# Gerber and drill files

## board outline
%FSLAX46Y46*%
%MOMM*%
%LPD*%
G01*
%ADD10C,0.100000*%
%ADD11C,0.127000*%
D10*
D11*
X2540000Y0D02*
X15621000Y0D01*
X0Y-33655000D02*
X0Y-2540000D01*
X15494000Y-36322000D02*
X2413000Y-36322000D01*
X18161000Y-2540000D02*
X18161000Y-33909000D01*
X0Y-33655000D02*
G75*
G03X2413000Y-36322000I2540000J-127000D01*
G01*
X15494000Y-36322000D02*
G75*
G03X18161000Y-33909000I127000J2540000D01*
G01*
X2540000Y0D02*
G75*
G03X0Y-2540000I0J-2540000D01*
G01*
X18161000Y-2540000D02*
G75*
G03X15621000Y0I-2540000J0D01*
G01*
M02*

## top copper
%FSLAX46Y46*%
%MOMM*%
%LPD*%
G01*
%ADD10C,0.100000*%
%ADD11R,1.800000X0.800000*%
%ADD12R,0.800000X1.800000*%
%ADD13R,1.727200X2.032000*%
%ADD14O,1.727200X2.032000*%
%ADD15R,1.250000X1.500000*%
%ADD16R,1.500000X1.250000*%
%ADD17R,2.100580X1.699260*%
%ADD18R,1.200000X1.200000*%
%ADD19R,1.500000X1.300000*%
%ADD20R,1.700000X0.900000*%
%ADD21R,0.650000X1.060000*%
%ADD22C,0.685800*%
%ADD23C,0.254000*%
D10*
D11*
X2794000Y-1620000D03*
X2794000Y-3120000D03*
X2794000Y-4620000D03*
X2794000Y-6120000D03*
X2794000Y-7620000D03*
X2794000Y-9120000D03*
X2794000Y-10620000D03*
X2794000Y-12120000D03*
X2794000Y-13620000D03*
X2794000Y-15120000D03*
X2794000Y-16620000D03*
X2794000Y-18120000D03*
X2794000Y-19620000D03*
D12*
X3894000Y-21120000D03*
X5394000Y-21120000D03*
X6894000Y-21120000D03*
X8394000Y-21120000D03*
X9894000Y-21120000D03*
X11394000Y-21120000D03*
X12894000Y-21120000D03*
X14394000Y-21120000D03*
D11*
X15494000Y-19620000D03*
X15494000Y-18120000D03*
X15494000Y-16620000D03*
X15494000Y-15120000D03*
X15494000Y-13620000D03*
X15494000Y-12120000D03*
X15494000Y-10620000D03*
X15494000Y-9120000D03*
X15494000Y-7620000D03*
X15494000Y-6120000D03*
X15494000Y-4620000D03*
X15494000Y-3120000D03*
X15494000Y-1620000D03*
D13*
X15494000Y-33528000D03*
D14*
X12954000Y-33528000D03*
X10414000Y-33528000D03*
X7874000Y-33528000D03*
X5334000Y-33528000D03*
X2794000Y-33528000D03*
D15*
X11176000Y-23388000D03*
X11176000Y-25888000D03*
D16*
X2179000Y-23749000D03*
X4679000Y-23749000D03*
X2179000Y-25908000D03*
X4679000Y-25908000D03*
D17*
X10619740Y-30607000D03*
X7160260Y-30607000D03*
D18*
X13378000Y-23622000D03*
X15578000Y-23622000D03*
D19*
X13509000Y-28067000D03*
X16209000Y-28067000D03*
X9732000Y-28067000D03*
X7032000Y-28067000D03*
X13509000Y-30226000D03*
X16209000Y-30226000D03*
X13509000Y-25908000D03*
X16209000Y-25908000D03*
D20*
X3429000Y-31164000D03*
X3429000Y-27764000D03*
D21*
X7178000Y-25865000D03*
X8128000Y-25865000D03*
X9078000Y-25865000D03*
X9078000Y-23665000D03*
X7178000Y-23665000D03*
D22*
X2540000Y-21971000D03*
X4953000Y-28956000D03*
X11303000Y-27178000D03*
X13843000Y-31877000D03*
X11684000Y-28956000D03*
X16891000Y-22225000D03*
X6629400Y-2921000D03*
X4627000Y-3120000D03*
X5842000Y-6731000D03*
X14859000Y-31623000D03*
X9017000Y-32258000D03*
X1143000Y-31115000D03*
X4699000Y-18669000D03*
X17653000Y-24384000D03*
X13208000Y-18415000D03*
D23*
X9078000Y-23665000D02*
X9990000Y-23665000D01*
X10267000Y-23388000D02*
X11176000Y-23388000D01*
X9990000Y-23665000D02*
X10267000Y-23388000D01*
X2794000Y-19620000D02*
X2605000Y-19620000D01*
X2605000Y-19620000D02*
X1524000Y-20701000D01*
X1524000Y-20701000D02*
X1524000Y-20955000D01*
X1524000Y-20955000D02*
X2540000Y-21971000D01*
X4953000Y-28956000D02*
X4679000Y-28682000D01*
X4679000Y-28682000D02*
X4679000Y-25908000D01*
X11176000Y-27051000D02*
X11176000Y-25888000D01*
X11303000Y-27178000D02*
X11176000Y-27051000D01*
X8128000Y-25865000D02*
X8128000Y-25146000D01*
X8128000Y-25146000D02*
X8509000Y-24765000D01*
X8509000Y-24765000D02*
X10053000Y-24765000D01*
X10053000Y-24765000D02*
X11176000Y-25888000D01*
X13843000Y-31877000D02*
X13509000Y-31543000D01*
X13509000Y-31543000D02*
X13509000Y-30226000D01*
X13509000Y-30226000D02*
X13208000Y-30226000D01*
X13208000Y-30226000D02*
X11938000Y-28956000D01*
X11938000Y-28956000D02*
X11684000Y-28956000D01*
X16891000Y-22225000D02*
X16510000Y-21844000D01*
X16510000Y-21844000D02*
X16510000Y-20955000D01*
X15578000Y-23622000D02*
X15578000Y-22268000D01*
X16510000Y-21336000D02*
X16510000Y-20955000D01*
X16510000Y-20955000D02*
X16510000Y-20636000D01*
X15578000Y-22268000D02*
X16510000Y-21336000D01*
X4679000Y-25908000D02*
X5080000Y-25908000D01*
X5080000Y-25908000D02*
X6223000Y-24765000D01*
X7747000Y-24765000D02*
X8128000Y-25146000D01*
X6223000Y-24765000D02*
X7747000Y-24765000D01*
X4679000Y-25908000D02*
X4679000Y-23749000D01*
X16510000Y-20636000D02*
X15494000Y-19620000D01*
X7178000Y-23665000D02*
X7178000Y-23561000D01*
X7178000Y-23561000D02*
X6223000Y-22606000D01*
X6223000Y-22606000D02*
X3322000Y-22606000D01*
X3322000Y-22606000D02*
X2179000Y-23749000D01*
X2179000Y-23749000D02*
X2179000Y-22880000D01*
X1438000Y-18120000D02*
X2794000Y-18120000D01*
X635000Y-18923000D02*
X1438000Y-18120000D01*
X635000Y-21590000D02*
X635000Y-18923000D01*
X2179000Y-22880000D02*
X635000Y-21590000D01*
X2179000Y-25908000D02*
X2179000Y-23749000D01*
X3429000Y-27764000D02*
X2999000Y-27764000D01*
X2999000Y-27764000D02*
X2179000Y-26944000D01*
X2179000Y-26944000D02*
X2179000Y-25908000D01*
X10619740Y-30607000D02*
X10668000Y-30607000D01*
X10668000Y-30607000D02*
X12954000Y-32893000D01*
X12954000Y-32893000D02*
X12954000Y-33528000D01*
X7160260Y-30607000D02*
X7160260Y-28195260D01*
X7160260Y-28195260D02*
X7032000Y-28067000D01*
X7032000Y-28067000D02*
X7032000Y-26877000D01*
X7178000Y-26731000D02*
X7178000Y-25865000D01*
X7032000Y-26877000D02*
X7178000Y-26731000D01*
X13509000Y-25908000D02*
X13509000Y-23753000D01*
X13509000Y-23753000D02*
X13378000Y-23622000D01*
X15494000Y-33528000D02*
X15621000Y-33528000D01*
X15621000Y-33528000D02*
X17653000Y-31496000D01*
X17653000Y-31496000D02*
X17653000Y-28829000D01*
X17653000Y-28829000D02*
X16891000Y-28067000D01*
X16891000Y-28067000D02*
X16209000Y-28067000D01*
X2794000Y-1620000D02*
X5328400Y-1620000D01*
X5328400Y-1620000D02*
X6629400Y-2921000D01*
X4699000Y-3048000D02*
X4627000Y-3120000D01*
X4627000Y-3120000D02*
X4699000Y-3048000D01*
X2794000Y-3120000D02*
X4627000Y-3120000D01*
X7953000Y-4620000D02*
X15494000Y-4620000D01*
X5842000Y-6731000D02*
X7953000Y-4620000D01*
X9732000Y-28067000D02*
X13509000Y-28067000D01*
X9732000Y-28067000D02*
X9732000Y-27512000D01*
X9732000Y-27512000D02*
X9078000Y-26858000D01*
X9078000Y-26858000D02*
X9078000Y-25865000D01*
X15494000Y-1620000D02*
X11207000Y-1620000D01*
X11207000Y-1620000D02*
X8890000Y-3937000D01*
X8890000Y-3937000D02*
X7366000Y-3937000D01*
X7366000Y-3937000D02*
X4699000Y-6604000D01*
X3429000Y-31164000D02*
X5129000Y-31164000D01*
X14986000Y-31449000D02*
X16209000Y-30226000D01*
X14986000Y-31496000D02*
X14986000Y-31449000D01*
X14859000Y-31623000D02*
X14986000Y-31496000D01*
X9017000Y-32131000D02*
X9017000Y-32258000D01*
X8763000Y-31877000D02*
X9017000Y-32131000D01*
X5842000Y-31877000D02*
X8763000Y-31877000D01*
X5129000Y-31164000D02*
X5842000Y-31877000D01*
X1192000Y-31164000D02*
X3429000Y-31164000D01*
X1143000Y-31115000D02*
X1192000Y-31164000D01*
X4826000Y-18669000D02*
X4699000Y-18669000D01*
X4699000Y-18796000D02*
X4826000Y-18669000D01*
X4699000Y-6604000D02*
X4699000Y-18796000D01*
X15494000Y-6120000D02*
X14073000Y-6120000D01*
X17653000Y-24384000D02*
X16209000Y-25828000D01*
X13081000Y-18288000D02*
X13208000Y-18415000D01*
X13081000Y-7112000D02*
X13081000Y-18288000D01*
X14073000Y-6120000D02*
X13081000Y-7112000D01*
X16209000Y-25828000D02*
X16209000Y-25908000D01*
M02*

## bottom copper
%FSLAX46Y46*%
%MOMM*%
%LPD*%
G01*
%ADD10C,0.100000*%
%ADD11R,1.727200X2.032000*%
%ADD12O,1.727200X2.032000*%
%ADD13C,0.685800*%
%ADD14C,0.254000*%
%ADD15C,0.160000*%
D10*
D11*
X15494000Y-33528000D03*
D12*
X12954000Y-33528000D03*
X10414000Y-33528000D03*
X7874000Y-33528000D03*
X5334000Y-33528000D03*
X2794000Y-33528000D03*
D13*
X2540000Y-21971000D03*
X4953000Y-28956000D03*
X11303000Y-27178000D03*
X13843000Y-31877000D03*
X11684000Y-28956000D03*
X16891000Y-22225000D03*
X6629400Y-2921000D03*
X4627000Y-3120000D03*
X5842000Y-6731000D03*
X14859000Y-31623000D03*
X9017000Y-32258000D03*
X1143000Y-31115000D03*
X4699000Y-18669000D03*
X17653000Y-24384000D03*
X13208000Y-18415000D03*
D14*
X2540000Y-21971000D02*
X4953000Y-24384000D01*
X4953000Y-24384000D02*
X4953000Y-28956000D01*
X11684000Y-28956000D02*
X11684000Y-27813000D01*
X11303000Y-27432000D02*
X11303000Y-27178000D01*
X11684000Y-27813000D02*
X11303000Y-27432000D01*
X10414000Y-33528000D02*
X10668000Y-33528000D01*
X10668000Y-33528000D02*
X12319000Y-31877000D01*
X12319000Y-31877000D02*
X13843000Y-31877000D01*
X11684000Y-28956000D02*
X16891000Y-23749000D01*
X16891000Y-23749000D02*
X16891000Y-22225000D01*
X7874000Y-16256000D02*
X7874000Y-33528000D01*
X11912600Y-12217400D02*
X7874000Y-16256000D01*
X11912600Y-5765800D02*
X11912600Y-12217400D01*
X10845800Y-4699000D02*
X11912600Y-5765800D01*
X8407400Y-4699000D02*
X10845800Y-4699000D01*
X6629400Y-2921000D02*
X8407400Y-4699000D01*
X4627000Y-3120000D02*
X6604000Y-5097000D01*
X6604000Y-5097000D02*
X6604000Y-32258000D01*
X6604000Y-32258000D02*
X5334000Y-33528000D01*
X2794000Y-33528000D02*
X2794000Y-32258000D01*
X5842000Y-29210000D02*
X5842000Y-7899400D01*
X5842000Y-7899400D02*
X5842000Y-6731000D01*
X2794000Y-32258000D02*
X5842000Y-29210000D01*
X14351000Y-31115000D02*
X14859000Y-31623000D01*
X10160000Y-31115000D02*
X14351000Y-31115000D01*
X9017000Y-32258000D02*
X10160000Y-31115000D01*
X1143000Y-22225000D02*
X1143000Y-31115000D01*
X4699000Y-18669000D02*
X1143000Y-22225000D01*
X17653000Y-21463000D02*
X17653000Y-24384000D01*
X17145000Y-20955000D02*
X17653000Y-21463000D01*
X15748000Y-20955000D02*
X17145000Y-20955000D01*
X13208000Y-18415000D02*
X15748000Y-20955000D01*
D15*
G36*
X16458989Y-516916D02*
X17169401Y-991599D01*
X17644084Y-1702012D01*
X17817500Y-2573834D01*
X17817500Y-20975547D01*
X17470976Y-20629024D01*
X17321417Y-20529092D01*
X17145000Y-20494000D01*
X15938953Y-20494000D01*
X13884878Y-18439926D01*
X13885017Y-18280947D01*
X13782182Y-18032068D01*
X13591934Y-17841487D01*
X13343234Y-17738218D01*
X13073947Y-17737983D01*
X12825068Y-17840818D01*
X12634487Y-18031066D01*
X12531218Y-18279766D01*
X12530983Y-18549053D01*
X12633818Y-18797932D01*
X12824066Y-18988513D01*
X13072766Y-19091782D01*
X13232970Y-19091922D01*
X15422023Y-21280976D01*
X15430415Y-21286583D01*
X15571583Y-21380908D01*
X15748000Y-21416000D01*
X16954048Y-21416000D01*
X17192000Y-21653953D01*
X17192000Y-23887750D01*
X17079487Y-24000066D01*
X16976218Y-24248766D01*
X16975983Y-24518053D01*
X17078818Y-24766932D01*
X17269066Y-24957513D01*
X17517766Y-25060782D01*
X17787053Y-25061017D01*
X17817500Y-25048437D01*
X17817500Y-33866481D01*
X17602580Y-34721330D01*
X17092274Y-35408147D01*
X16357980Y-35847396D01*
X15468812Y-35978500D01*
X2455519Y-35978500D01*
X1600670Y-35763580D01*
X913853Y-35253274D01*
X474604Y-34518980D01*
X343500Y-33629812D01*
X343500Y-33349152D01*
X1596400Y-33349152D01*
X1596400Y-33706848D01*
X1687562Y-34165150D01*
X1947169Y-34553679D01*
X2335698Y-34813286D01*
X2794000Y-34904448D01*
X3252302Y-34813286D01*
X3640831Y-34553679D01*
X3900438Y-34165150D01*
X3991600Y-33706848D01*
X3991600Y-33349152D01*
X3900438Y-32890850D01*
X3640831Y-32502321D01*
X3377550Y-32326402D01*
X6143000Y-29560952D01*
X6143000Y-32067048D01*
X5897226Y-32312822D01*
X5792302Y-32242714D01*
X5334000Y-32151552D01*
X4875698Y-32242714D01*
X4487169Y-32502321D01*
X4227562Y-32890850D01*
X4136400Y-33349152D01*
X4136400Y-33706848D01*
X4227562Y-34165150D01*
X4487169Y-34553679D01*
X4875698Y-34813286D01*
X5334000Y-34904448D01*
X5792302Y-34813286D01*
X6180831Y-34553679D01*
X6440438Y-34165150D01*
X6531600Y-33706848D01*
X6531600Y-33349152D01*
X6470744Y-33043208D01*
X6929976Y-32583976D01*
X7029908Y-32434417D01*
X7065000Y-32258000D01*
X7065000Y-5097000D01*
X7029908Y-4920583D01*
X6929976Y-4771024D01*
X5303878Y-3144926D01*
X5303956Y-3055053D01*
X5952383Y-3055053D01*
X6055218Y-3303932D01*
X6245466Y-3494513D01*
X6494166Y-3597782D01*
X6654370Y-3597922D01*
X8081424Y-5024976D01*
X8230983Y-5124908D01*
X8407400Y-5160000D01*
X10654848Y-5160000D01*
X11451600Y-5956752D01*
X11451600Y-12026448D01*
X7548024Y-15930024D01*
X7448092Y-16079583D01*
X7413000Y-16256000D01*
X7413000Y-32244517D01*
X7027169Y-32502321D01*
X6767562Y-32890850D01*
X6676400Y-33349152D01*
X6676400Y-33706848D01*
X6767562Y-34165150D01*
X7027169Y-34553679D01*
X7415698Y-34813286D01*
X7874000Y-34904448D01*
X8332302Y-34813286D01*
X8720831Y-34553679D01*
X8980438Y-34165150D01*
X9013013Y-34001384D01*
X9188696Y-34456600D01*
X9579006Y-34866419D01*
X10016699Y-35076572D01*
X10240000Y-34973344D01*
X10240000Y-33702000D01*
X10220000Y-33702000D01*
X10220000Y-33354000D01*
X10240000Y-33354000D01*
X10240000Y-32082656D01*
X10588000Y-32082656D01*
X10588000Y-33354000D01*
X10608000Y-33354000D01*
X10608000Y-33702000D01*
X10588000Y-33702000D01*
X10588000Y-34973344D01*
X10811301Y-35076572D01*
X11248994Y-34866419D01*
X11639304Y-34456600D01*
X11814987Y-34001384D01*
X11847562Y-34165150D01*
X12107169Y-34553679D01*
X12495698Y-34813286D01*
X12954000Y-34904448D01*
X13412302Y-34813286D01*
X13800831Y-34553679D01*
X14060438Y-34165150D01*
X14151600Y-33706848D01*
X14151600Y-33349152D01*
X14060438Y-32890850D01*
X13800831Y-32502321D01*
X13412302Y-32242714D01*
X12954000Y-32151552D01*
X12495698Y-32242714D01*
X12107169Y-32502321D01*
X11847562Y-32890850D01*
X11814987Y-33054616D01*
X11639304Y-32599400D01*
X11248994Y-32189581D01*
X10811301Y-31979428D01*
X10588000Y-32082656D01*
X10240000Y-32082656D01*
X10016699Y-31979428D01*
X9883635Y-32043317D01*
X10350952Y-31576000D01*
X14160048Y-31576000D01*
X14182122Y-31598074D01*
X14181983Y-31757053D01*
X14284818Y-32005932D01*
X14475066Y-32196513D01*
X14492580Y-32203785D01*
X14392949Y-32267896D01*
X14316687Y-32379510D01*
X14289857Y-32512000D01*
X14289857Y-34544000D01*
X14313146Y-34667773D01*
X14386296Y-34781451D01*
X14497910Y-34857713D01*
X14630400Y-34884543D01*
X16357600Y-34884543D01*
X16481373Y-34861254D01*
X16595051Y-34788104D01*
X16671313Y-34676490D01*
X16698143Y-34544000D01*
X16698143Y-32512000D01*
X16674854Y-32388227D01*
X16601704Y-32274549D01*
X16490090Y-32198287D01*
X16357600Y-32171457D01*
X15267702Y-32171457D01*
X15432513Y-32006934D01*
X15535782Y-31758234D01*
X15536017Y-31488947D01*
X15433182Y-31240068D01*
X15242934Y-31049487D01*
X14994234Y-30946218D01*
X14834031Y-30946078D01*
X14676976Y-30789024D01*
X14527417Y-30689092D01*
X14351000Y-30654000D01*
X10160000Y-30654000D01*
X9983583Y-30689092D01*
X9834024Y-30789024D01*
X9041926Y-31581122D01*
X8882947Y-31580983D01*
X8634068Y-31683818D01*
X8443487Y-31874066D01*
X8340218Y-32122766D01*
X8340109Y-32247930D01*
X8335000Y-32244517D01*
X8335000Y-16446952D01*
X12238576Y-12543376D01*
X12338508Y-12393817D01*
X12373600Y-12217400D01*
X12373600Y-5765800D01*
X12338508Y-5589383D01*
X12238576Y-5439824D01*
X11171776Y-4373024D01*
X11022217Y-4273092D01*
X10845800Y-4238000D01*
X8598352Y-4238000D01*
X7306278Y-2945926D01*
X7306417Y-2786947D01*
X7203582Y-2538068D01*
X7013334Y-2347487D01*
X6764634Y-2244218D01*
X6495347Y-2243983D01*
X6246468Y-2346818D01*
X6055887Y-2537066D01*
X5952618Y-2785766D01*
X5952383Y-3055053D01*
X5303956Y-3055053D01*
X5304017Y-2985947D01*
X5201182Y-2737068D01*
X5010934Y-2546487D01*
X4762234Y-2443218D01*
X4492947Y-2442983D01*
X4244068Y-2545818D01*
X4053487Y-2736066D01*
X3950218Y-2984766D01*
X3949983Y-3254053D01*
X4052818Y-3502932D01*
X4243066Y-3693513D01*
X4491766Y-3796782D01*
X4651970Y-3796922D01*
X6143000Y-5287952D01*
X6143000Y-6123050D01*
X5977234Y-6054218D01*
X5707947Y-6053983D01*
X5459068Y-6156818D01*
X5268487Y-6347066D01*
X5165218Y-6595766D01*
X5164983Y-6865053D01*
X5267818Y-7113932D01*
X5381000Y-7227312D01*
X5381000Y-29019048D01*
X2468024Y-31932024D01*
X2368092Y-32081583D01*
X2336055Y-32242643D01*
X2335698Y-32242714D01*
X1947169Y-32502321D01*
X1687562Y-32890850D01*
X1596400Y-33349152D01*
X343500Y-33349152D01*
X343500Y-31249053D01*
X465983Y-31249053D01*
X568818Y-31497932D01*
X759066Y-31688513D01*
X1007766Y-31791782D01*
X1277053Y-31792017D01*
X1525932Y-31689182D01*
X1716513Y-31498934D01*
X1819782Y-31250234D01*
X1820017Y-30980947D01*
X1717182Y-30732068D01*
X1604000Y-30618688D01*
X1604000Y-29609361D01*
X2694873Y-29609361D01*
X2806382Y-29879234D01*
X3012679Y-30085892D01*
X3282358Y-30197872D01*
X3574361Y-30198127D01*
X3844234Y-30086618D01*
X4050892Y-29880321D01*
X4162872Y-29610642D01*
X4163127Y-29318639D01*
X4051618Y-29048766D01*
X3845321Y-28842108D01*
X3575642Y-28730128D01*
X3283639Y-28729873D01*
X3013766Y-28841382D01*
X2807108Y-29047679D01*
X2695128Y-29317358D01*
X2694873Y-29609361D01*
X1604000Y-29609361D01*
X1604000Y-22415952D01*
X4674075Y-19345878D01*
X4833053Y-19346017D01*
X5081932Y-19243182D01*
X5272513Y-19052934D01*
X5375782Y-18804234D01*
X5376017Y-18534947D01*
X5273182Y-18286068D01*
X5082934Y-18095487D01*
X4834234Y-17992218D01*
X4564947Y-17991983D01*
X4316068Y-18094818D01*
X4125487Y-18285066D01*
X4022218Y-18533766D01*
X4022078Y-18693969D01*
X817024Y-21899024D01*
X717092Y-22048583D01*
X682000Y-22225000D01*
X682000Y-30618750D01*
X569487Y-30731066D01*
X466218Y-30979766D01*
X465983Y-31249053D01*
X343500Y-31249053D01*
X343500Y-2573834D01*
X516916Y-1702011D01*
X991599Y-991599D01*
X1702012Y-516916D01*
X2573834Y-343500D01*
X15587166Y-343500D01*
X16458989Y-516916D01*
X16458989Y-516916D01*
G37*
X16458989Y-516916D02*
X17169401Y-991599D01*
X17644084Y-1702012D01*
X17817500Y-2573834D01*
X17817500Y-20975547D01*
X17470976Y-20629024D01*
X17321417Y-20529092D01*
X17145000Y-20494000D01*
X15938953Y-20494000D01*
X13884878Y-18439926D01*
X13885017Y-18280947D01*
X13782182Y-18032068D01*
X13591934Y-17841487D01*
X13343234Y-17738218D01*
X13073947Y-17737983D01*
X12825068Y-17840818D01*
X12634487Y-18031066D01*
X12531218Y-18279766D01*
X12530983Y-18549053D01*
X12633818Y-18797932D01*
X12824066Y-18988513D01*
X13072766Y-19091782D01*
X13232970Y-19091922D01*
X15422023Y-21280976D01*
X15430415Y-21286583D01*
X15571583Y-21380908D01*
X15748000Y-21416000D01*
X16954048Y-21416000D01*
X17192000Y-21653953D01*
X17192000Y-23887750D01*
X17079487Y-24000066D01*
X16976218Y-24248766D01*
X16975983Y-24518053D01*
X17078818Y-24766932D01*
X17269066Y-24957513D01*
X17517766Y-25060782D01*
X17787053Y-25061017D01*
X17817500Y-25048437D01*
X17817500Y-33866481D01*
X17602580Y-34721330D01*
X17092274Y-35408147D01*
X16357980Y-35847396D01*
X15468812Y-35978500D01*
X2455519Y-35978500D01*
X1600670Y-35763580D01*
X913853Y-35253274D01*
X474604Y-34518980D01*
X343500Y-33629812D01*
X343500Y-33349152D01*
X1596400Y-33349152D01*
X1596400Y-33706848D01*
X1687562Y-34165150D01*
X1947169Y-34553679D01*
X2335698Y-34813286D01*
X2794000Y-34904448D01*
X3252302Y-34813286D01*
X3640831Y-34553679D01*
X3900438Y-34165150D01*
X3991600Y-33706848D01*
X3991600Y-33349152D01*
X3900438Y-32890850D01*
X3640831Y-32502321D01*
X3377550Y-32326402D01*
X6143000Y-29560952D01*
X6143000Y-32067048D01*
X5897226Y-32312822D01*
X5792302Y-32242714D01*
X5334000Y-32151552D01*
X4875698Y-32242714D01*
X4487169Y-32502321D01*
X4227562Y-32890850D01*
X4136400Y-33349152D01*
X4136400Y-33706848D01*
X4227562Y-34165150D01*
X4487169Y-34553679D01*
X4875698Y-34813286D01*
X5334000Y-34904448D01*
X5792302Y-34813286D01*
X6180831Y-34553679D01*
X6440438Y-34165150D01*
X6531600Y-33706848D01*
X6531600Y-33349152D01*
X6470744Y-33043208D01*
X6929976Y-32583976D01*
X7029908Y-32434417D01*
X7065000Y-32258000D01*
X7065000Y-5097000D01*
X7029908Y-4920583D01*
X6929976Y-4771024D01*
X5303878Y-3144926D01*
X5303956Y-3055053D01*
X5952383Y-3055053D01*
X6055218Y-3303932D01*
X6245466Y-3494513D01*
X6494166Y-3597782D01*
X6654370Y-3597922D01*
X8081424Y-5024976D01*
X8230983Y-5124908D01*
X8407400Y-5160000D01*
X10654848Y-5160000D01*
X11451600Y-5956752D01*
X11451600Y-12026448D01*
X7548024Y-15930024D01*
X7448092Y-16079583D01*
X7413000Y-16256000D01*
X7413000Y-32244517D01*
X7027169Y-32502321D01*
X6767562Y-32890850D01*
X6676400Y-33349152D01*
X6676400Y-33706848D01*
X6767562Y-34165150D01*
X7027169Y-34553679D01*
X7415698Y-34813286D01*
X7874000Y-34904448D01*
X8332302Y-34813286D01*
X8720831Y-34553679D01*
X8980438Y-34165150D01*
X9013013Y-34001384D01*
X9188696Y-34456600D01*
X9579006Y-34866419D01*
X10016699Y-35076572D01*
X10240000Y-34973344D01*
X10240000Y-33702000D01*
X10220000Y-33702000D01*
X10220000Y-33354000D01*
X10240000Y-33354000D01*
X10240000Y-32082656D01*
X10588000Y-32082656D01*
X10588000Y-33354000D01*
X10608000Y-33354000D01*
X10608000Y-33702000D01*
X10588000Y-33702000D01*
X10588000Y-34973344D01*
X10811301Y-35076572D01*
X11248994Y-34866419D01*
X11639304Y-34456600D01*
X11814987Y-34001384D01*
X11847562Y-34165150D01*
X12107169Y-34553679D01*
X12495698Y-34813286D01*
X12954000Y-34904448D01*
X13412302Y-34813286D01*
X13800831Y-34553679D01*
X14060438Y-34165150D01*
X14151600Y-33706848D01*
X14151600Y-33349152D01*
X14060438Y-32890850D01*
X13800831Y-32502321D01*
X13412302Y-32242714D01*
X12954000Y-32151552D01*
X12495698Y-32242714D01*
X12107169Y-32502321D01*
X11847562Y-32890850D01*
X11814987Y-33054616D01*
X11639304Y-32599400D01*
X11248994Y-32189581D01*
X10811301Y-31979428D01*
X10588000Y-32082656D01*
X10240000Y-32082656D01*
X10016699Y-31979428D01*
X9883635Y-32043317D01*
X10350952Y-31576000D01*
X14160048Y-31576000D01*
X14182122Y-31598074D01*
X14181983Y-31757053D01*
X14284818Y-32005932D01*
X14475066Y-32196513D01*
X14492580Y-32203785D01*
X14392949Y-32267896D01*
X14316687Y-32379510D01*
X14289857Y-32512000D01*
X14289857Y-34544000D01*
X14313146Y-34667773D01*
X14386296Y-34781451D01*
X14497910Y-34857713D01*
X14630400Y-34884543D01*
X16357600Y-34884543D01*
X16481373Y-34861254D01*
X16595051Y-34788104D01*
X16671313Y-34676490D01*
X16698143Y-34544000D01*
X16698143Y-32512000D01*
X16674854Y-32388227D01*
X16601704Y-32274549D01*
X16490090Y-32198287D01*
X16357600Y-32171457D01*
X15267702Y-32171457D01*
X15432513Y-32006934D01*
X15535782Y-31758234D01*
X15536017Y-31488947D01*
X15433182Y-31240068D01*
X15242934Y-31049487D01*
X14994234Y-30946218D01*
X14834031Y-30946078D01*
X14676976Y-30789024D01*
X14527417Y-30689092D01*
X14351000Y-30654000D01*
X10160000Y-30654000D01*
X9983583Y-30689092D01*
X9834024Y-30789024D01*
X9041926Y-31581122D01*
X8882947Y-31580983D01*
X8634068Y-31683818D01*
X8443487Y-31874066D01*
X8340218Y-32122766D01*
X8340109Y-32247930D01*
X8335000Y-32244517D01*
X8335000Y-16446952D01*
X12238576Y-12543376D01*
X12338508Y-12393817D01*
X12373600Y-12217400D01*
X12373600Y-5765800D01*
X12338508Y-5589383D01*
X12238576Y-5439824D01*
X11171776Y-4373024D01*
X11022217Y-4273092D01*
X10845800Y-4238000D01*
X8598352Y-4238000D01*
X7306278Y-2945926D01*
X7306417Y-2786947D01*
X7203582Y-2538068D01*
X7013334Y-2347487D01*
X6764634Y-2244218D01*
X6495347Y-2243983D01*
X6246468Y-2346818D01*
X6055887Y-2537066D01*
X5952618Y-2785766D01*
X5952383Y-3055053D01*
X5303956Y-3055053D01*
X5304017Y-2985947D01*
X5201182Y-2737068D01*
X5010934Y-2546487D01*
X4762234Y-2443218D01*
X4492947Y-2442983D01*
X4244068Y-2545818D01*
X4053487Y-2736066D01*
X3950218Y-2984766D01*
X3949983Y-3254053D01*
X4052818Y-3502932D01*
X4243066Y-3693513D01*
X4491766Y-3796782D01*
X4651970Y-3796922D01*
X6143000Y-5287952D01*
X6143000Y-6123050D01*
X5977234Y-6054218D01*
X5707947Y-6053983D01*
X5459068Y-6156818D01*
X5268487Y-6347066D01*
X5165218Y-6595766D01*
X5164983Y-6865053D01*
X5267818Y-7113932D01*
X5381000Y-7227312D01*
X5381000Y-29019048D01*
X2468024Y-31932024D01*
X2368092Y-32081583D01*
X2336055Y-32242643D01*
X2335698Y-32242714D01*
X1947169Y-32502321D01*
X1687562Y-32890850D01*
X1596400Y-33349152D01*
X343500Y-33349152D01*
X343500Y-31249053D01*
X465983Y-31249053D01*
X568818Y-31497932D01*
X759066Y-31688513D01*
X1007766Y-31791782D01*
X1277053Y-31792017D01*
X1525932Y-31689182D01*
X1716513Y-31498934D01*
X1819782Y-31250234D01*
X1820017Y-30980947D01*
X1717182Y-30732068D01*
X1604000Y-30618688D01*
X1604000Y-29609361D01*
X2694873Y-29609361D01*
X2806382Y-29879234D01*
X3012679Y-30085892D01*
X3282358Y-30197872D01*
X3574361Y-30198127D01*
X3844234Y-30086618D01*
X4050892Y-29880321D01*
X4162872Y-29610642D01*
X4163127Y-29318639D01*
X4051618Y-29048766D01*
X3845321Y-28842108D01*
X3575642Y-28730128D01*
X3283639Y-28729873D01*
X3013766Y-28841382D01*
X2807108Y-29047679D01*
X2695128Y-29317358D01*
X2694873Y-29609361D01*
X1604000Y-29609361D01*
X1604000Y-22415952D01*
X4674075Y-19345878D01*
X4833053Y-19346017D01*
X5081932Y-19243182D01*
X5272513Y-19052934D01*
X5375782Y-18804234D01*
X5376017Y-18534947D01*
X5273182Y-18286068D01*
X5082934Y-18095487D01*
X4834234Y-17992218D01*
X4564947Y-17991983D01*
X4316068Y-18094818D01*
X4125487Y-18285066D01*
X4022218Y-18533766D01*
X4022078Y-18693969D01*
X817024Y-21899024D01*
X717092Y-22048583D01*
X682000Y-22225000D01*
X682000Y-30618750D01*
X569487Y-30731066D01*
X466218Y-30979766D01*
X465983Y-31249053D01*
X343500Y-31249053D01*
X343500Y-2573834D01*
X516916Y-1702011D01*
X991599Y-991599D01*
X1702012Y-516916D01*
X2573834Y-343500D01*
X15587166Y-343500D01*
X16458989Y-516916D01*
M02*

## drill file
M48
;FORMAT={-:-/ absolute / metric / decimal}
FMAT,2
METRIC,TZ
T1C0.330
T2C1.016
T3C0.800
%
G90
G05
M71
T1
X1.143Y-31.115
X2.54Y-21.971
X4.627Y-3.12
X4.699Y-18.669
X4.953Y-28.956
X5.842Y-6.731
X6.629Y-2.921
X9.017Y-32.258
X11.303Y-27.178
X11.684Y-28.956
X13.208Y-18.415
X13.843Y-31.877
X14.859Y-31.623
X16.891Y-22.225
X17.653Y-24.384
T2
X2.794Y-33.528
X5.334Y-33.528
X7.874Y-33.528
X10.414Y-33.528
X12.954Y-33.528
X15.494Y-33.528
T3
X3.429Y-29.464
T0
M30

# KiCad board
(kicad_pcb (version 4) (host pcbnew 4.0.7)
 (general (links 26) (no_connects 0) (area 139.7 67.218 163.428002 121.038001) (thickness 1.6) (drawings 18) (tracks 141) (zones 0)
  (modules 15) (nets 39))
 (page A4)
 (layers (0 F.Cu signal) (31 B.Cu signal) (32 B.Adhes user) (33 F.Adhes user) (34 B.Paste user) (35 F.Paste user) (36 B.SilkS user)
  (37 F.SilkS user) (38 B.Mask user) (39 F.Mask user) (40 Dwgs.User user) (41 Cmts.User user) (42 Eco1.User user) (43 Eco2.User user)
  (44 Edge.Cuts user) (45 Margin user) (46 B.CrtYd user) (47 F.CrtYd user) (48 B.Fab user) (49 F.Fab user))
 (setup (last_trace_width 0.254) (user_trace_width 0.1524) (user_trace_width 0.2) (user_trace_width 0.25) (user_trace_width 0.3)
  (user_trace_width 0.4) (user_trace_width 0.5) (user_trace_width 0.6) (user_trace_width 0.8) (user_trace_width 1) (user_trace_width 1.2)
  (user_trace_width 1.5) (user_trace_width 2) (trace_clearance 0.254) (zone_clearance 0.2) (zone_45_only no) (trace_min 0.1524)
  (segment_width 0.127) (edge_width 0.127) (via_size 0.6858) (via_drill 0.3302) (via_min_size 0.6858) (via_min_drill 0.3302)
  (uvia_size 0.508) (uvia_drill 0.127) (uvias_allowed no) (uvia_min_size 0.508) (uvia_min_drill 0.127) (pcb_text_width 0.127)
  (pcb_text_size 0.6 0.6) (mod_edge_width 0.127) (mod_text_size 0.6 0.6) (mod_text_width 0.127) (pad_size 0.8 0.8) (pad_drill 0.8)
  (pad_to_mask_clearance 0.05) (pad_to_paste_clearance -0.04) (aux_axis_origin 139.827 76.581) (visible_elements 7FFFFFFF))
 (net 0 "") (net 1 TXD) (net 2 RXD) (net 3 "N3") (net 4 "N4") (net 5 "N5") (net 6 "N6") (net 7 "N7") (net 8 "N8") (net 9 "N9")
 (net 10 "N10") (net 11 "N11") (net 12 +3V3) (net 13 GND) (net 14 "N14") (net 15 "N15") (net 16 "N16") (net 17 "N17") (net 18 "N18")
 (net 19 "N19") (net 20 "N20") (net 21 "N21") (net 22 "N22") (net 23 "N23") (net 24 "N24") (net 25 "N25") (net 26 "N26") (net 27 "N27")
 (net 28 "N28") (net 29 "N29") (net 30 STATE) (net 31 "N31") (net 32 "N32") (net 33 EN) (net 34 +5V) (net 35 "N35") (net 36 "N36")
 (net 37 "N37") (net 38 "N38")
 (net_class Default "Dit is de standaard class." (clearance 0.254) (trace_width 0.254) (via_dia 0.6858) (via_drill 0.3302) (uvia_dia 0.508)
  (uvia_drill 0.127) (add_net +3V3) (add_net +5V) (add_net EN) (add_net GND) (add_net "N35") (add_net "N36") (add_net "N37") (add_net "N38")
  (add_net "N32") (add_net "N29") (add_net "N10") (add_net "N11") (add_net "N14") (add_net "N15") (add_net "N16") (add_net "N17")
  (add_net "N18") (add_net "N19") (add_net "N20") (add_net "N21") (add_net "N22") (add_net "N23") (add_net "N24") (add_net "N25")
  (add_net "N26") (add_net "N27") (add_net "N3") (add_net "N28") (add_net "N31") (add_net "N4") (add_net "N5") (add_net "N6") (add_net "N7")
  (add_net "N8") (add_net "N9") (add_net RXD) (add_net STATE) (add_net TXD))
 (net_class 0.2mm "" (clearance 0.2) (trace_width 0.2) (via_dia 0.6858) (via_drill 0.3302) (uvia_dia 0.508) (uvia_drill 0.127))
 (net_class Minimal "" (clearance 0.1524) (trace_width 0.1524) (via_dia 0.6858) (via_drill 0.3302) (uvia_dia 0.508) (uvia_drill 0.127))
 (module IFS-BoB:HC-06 (layer F.Cu) (at 148.971 84.201)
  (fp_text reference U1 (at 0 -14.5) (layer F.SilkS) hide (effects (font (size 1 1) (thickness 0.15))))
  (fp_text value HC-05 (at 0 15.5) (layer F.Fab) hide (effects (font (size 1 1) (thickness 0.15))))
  (pad 1 smd rect (at -6.35 -6) (size 1.8 0.8) (layers F.Cu F.Paste F.Mask) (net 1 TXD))
  (pad 2 smd rect (at -6.35 -4.5) (size 1.8 0.8) (layers F.Cu F.Paste F.Mask) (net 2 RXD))
  (pad 3 smd rect (at -6.35 -3) (size 1.8 0.8) (layers F.Cu F.Paste F.Mask) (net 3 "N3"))
  (pad 4 smd rect (at -6.35 -1.5) (size 1.8 0.8) (layers F.Cu F.Paste F.Mask) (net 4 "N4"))
  (pad 5 smd rect (at -6.35 0) (size 1.8 0.8) (layers F.Cu F.Paste F.Mask) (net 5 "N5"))
  (pad 6 smd rect (at -6.35 1.5) (size 1.8 0.8) (layers F.Cu F.Paste F.Mask) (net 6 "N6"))
  (pad 7 smd rect (at -6.35 3) (size 1.8 0.8) (layers F.Cu F.Paste F.Mask) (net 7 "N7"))
  (pad 8 smd rect (at -6.35 4.5) (size 1.8 0.8) (layers F.Cu F.Paste F.Mask) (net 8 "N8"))
  (pad 9 smd rect (at -6.35 6) (size 1.8 0.8) (layers F.Cu F.Paste F.Mask) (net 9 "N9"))
  (pad 10 smd rect (at -6.35 7.5) (size 1.8 0.8) (layers F.Cu F.Paste F.Mask) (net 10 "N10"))
  (pad 11 smd rect (at -6.35 9) (size 1.8 0.8) (layers F.Cu F.Paste F.Mask) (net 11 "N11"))
  (pad 12 smd rect (at -6.35 10.5) (size 1.8 0.8) (layers F.Cu F.Paste F.Mask) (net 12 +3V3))
  (pad 13 smd rect (at -6.35 12) (size 1.8 0.8) (layers F.Cu F.Paste F.Mask) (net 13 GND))
  (pad 14 smd rect (at -5.25 13.5) (size 0.8 1.8) (layers F.Cu F.Paste F.Mask) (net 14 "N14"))
  (pad 15 smd rect (at -3.75 13.5) (size 0.8 1.8) (layers F.Cu F.Paste F.Mask) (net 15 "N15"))
  (pad 16 smd rect (at -2.25 13.5) (size 0.8 1.8) (layers F.Cu F.Paste F.Mask) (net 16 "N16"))
  (pad 17 smd rect (at -0.75 13.5) (size 0.8 1.8) (layers F.Cu F.Paste F.Mask) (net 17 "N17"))
  (pad 18 smd rect (at 0.75 13.5) (size 0.8 1.8) (layers F.Cu F.Paste F.Mask))
  (pad 19 smd rect (at 2.25 13.5) (size 0.8 1.8) (layers F.Cu F.Paste F.Mask) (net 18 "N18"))
  (pad 20 smd rect (at 3.75 13.5) (size 0.8 1.8) (layers F.Cu F.Paste F.Mask) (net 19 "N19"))
  (pad 21 smd rect (at 5.25 13.5) (size 0.8 1.8) (layers F.Cu F.Paste F.Mask) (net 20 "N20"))
  (pad 22 smd rect (at 6.35 12) (size 1.8 0.8) (layers F.Cu F.Paste F.Mask) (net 13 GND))
  (pad 23 smd rect (at 6.35 10.5) (size 1.8 0.8) (layers F.Cu F.Paste F.Mask) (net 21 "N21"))
  (pad 24 smd rect (at 6.35 9) (size 1.8 0.8) (layers F.Cu F.Paste F.Mask) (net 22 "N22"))
  (pad 25 smd rect (at 6.35 7.5) (size 1.8 0.8) (layers F.Cu F.Paste F.Mask) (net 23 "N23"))
  (pad 26 smd rect (at 6.35 6) (size 1.8 0.8) (layers F.Cu F.Paste F.Mask) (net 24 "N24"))
  (pad 27 smd rect (at 6.35 4.5) (size 1.8 0.8) (layers F.Cu F.Paste F.Mask) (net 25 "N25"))
  (pad 28 smd rect (at 6.35 3) (size 1.8 0.8) (layers F.Cu F.Paste F.Mask) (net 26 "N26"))
  (pad 29 smd rect (at 6.35 1.5) (size 1.8 0.8) (layers F.Cu F.Paste F.Mask) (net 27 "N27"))
  (pad 30 smd rect (at 6.35 0) (size 1.8 0.8) (layers F.Cu F.Paste F.Mask) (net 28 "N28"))
  (pad 31 smd rect (at 6.35 -1.5) (size 1.8 0.8) (layers F.Cu F.Paste F.Mask) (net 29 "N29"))
  (pad 32 smd rect (at 6.35 -3) (size 1.8 0.8) (layers F.Cu F.Paste F.Mask) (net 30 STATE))
  (pad 33 smd rect (at 6.35 -4.5) (size 1.8 0.8) (layers F.Cu F.Paste F.Mask) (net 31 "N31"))
  (pad 34 smd rect (at 6.35 -6) (size 1.8 0.8) (layers F.Cu F.Paste F.Mask) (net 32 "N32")))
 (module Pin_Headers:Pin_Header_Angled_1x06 (layer F.Cu) (at 155.321 110.109 270)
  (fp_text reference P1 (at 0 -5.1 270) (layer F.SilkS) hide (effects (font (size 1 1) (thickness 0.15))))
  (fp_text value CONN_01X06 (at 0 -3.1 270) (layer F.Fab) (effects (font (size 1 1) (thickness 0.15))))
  (pad 1 thru_hole rect (at 0 0 270) (size 2.032 1.7272) (drill 1.016) (layers *.Cu *.Mask) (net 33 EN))
  (pad 2 thru_hole oval (at 0 2.54 270) (size 2.032 1.7272) (drill 1.016) (layers *.Cu *.Mask) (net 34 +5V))
  (pad 3 thru_hole oval (at 0 5.08 270) (size 2.032 1.7272) (drill 1.016) (layers *.Cu *.Mask) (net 13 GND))
  (pad 4 thru_hole oval (at 0 7.62 270) (size 2.032 1.7272) (drill 1.016) (layers *.Cu *.Mask) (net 1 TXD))
  (pad 5 thru_hole oval (at 0 10.16 270) (size 2.032 1.7272) (drill 1.016) (layers *.Cu *.Mask) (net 2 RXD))
  (pad 6 thru_hole oval (at 0 12.7 270) (size 2.032 1.7272) (drill 1.016) (layers *.Cu *.Mask) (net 30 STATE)))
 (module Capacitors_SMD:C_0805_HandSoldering (layer F.Cu) (at 151.003 101.219 270)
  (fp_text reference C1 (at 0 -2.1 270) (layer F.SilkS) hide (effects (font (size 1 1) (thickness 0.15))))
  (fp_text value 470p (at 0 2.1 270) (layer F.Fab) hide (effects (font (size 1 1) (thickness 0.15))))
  (pad 1 smd rect (at -1.25 0 270) (size 1.5 1.25) (layers F.Cu F.Paste F.Mask) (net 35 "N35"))
  (pad 2 smd rect (at 1.25 0 270) (size 1.5 1.25) (layers F.Cu F.Paste F.Mask) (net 13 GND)))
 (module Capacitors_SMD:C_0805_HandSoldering (layer F.Cu) (at 143.256 100.33)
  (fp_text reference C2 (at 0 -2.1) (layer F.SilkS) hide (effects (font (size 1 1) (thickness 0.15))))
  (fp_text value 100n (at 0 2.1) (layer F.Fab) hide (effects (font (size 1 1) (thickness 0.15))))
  (pad 1 smd rect (at -1.25 0) (size 1.5 1.25) (layers F.Cu F.Paste F.Mask) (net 12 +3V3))
  (pad 2 smd rect (at 1.25 0) (size 1.5 1.25) (layers F.Cu F.Paste F.Mask) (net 13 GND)))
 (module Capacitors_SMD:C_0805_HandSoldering (layer F.Cu) (at 143.256 102.489)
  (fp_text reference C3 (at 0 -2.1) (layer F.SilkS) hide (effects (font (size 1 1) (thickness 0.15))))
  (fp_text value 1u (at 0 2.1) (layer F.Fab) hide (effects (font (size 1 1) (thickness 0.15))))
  (pad 1 smd rect (at -1.25 0) (size 1.5 1.25) (layers F.Cu F.Paste F.Mask) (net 12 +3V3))
  (pad 2 smd rect (at 1.25 0) (size 1.5 1.25) (layers F.Cu F.Paste F.Mask) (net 13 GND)))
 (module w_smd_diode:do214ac (layer F.Cu) (at 148.717 107.188)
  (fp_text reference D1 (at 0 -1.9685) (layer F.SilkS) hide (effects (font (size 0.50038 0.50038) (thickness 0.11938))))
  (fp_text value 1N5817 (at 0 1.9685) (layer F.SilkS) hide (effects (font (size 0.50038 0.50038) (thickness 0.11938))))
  (pad 2 smd rect (at 1.72974 0) (size 2.10058 1.69926) (layers F.Cu F.Paste F.Mask) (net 34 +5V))
  (pad 1 smd rect (at -1.72974 0) (size 2.10058 1.69926) (layers F.Cu F.Paste F.Mask) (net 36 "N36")))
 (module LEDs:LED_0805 (layer F.Cu) (at 154.305 100.203 180)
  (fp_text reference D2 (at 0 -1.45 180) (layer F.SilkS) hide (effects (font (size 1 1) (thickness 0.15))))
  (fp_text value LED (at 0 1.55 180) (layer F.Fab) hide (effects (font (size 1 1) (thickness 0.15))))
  (pad 2 smd rect (at 1.1 0) (size 1.2 1.2) (layers F.Cu F.Paste F.Mask) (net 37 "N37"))
  (pad 1 smd rect (at -1.1 0) (size 1.2 1.2) (layers F.Cu F.Paste F.Mask) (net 13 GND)))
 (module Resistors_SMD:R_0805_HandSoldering (layer F.Cu) (at 154.686 104.648)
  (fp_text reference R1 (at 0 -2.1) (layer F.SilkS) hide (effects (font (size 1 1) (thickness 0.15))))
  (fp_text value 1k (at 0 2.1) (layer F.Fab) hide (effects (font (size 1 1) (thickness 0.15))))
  (pad 1 smd rect (at -1.35 0) (size 1.5 1.3) (layers F.Cu F.Paste F.Mask) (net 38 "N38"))
  (pad 2 smd rect (at 1.35 0) (size 1.5 1.3) (layers F.Cu F.Paste F.Mask) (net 33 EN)))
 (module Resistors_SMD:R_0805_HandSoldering (layer F.Cu) (at 148.209 104.648 180)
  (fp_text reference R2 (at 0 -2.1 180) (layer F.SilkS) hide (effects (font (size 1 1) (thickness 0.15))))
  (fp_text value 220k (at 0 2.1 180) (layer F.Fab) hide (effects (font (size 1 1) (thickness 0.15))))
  (pad 1 smd rect (at -1.35 0 180) (size 1.5 1.3) (layers F.Cu F.Paste F.Mask) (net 38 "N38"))
  (pad 2 smd rect (at 1.35 0 180) (size 1.5 1.3) (layers F.Cu F.Paste F.Mask) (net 36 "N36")))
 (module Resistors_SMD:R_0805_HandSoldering (layer F.Cu) (at 154.686 106.807)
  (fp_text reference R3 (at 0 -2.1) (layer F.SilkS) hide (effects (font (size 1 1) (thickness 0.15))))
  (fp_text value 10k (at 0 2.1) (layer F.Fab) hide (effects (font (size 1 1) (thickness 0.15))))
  (pad 1 smd rect (at -1.35 0) (size 1.5 1.3) (layers F.Cu F.Paste F.Mask) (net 13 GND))
  (pad 2 smd rect (at 1.35 0) (size 1.5 1.3) (layers F.Cu F.Paste F.Mask) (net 32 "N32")))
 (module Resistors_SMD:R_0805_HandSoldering (layer F.Cu) (at 154.686 102.489)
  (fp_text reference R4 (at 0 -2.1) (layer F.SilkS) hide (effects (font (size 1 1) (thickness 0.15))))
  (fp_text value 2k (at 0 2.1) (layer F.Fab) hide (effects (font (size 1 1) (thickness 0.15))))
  (pad 1 smd rect (at -1.35 0) (size 1.5 1.3) (layers F.Cu F.Paste F.Mask) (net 37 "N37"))
  (pad 2 smd rect (at 1.35 0) (size 1.5 1.3) (layers F.Cu F.Paste F.Mask) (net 29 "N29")))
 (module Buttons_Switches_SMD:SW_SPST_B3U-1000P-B (layer F.Cu) (at 143.256 106.045 90)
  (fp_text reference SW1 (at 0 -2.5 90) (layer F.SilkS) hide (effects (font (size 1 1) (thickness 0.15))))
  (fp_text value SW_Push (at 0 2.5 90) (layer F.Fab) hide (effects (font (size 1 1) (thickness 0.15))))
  (pad 1 smd rect (at -1.7 0 90) (size 0.9 1.7) (layers F.Cu F.Paste F.Mask) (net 32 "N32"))
  (pad 2 smd rect (at 1.7 0 90) (size 0.9 1.7) (layers F.Cu F.Paste F.Mask) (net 12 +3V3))
  (pad "" np_thru_hole circle (at 0 0 90) (size 0.8 0.8) (drill 0.8) (layers *.Cu *.Mask)))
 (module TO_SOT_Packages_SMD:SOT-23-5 (layer F.Cu) (at 147.955 101.346 90)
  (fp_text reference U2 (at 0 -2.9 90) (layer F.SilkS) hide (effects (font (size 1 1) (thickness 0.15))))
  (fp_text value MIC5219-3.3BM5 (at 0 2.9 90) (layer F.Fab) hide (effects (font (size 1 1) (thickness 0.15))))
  (pad 1 smd rect (at -1.1 -0.95 90) (size 1.06 0.65) (layers F.Cu F.Paste F.Mask) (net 36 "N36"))
  (pad 2 smd rect (at -1.1 0 90) (size 1.06 0.65) (layers F.Cu F.Paste F.Mask) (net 13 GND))
  (pad 3 smd rect (at -1.1 0.95 90) (size 1.06 0.65) (layers F.Cu F.Paste F.Mask) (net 38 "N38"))
  (pad 4 smd rect (at 1.1 0.95 90) (size 1.06 0.65) (layers F.Cu F.Paste F.Mask) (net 35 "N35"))
  (pad 5 smd rect (at 1.1 -0.95 90) (size 1.06 0.65) (layers F.Cu F.Paste F.Mask) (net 12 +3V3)))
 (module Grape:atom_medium (layer B.Cu) (at 148.9964 87.376 180)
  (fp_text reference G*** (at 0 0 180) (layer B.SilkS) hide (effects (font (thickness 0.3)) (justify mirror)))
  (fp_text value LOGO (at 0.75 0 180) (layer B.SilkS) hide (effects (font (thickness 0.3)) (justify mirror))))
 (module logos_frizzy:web (layer B.Cu) (at 148.9456 95.3897 180)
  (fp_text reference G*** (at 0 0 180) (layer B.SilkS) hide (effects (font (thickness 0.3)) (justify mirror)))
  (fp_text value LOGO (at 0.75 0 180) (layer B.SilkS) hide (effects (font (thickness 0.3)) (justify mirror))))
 (gr_line (start 142.367 76.581) (end 155.448 76.581) (angle 90) (layer Edge.Cuts) (width 0.127))
 (gr_line (start 139.827 110.236) (end 139.827 79.121) (angle 90) (layer Edge.Cuts) (width 0.127))
 (gr_line (start 155.321 112.903) (end 142.24 112.903) (angle 90) (layer Edge.Cuts) (width 0.127))
 (gr_line (start 157.988 79.121) (end 157.988 110.49) (angle 90) (layer Edge.Cuts) (width 0.127))
 (gr_arc (start 142.367 110.363) (end 142.24 112.903) (angle 90) (layer Edge.Cuts) (width 0.127))
 (gr_arc (start 155.448 110.363) (end 157.988 110.49) (angle 90) (layer Edge.Cuts) (width 0.127))
 (gr_arc (start 142.367 79.121) (end 139.827 79.121) (angle 90) (layer Edge.Cuts) (width 0.127))
 (gr_arc (start 155.448 79.121) (end 155.448 76.581) (angle 90) (layer Edge.Cuts) (width 0.127))
 (segment (start 148.905 100.246) (end 149.817 100.246) (width 0.254) (layer F.Cu) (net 35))
 (segment (start 150.094 99.969) (end 151.003 99.969) (width 0.254) (layer F.Cu) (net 35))
 (segment (start 149.817 100.246) (end 150.094 99.969) (width 0.254) (layer F.Cu) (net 35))
 (segment (start 142.621 96.201) (end 142.432 96.201) (width 0.254) (layer F.Cu) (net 13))
 (segment (start 142.432 96.201) (end 141.351 97.282) (width 0.254) (layer F.Cu) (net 13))
 (segment (start 141.351 97.282) (end 141.351 97.536) (width 0.254) (layer F.Cu) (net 13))
 (segment (start 141.351 97.536) (end 142.367 98.552) (width 0.254) (layer F.Cu) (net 13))
 (via (at 142.367 98.552) (size 0.6858) (drill 0.3302) (layers F.Cu B.Cu) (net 13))
 (segment (start 142.367 98.552) (end 144.78 100.965) (width 0.254) (layer B.Cu) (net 13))
 (segment (start 144.78 100.965) (end 144.78 105.537) (width 0.254) (layer B.Cu) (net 13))
 (via (at 144.78 105.537) (size 0.6858) (drill 0.3302) (layers F.Cu B.Cu) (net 13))
 (segment (start 144.78 105.537) (end 144.506 105.263) (width 0.254) (layer F.Cu) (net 13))
 (segment (start 144.506 105.263) (end 144.506 102.489) (width 0.254) (layer F.Cu) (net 13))
 (segment (start 151.511 105.537) (end 151.511 104.394) (width 0.254) (layer B.Cu) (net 13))
 (segment (start 151.003 103.632) (end 151.003 102.469) (width 0.254) (layer F.Cu) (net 13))
 (segment (start 151.13 103.759) (end 151.003 103.632) (width 0.254) (layer F.Cu) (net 13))
 (via (at 151.13 103.759) (size 0.6858) (drill 0.3302) (layers F.Cu B.Cu) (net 13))
 (segment (start 151.13 104.013) (end 151.13 103.759) (width 0.254) (layer B.Cu) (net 13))
 (segment (start 151.511 104.394) (end 151.13 104.013) (width 0.254) (layer B.Cu) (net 13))
 (segment (start 147.955 102.446) (end 147.955 101.727) (width 0.254) (layer F.Cu) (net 13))
 (segment (start 147.955 101.727) (end 148.336 101.346) (width 0.254) (layer F.Cu) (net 13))
 (segment (start 148.336 101.346) (end 149.88 101.346) (width 0.254) (layer F.Cu) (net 13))
 (segment (start 149.88 101.346) (end 151.003 102.469) (width 0.254) (layer F.Cu) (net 13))
 (segment (start 150.241 110.109) (end 150.495 110.109) (width 0.254) (layer B.Cu) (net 13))
 (segment (start 150.495 110.109) (end 152.146 108.458) (width 0.254) (layer B.Cu) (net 13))
 (segment (start 152.146 108.458) (end 153.67 108.458) (width 0.254) (layer B.Cu) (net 13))
 (via (at 153.67 108.458) (size 0.6858) (drill 0.3302) (layers F.Cu B.Cu) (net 13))
 (segment (start 153.67 108.458) (end 153.336 108.124) (width 0.254) (layer F.Cu) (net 13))
 (segment (start 153.336 108.124) (end 153.336 106.807) (width 0.254) (layer F.Cu) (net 13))
 (segment (start 153.336 106.807) (end 153.035 106.807) (width 0.254) (layer F.Cu) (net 13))
 (segment (start 153.035 106.807) (end 151.765 105.537) (width 0.254) (layer F.Cu) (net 13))
 (segment (start 151.765 105.537) (end 151.511 105.537) (width 0.254) (layer F.Cu) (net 13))
 (via (at 151.511 105.537) (size 0.6858) (drill 0.3302) (layers F.Cu B.Cu) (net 13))
 (segment (start 151.511 105.537) (end 156.718 100.33) (width 0.254) (layer B.Cu) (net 13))
 (segment (start 156.718 100.33) (end 156.718 98.806) (width 0.254) (layer B.Cu) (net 13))
 (via (at 156.718 98.806) (size 0.6858) (drill 0.3302) (layers F.Cu B.Cu) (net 13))
 (segment (start 156.718 98.806) (end 156.337 98.425) (width 0.254) (layer F.Cu) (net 13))
 (segment (start 156.337 98.425) (end 156.337 97.536) (width 0.254) (layer F.Cu) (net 13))
 (segment (start 155.405 100.203) (end 155.405 98.849) (width 0.254) (layer F.Cu) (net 13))
 (segment (start 156.337 97.917) (end 156.337 97.536) (width 0.254) (layer F.Cu) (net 13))
 (segment (start 156.337 97.536) (end 156.337 97.217) (width 0.254) (layer F.Cu) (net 13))
 (segment (start 155.405 98.849) (end 156.337 97.917) (width 0.254) (layer F.Cu) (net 13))
 (segment (start 144.506 102.489) (end 144.907 102.489) (width 0.254) (layer F.Cu) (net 13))
 (segment (start 144.907 102.489) (end 146.05 101.346) (width 0.254) (layer F.Cu) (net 13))
 (segment (start 147.574 101.346) (end 147.955 101.727) (width 0.254) (layer F.Cu) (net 13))
 (segment (start 146.05 101.346) (end 147.574 101.346) (width 0.254) (layer F.Cu) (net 13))
 (segment (start 144.506 102.489) (end 144.506 100.33) (width 0.254) (layer F.Cu) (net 13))
 (segment (start 156.337 97.217) (end 155.321 96.201) (width 0.254) (layer F.Cu) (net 13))
 (segment (start 147.005 100.246) (end 147.005 100.142) (width 0.254) (layer F.Cu) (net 12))
 (segment (start 147.005 100.142) (end 146.05 99.187) (width 0.254) (layer F.Cu) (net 12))
 (segment (start 146.05 99.187) (end 143.149 99.187) (width 0.254) (layer F.Cu) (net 12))
 (segment (start 143.149 99.187) (end 142.006 100.33) (width 0.254) (layer F.Cu) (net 12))
 (segment (start 142.006 100.33) (end 142.006 99.461) (width 0.254) (layer F.Cu) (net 12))
 (segment (start 141.265 94.701) (end 142.621 94.701) (width 0.254) (layer F.Cu) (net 12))
 (segment (start 140.462 95.504) (end 141.265 94.701) (width 0.254) (layer F.Cu) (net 12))
 (segment (start 140.462 98.171) (end 140.462 95.504) (width 0.254) (layer F.Cu) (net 12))
 (segment (start 142.006 99.461) (end 140.462 98.171) (width 0.254) (layer F.Cu) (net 12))
 (segment (start 142.006 102.489) (end 142.006 100.33) (width 0.254) (layer F.Cu) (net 12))
 (segment (start 143.256 104.345) (end 142.826 104.345) (width 0.254) (layer F.Cu) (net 12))
 (segment (start 142.826 104.345) (end 142.006 103.525) (width 0.254) (layer F.Cu) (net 12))
 (segment (start 142.006 103.525) (end 142.006 102.489) (width 0.254) (layer F.Cu) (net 12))
 (segment (start 150.44674 107.188) (end 150.495 107.188) (width 0.254) (layer F.Cu) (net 34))
 (segment (start 150.495 107.188) (end 152.781 109.474) (width 0.254) (layer F.Cu) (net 34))
 (segment (start 152.781 109.474) (end 152.781 110.109) (width 0.254) (layer F.Cu) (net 34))
 (segment (start 146.98726 107.188) (end 146.98726 104.77626) (width 0.254) (layer F.Cu) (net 36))
 (segment (start 146.98726 104.77626) (end 146.859 104.648) (width 0.254) (layer F.Cu) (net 36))
 (segment (start 146.859 104.648) (end 146.859 103.458) (width 0.254) (layer F.Cu) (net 36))
 (segment (start 147.005 103.312) (end 147.005 102.446) (width 0.254) (layer F.Cu) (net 36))
 (segment (start 146.859 103.458) (end 147.005 103.312) (width 0.254) (layer F.Cu) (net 36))
 (segment (start 153.336 102.489) (end 153.336 100.334) (width 0.254) (layer F.Cu) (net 37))
 (segment (start 153.336 100.334) (end 153.205 100.203) (width 0.254) (layer F.Cu) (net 37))
 (segment (start 155.321 110.109) (end 155.448 110.109) (width 0.254) (layer F.Cu) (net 33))
 (segment (start 155.448 110.109) (end 157.48 108.077) (width 0.254) (layer F.Cu) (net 33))
 (segment (start 157.48 108.077) (end 157.48 105.41) (width 0.254) (layer F.Cu) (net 33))
 (segment (start 157.48 105.41) (end 156.718 104.648) (width 0.254) (layer F.Cu) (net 33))
 (segment (start 156.718 104.648) (end 156.036 104.648) (width 0.254) (layer F.Cu) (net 33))
 (segment (start 142.621 78.201) (end 145.1554 78.201) (width 0.254) (layer F.Cu) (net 1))
 (segment (start 147.701 92.837) (end 147.701 110.109) (width 0.254) (layer B.Cu) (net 1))
 (segment (start 151.7396 88.7984) (end 147.701 92.837) (width 0.254) (layer B.Cu) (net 1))
 (segment (start 151.7396 82.3468) (end 151.7396 88.7984) (width 0.254) (layer B.Cu) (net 1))
 (segment (start 150.6728 81.28) (end 151.7396 82.3468) (width 0.254) (layer B.Cu) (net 1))
 (segment (start 148.2344 81.28) (end 150.6728 81.28) (width 0.254) (layer B.Cu) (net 1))
 (segment (start 146.4564 79.502) (end 148.2344 81.28) (width 0.254) (layer B.Cu) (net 1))
 (via (at 146.4564 79.502) (size 0.6858) (drill 0.3302) (layers F.Cu B.Cu) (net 1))
 (segment (start 145.1554 78.201) (end 146.4564 79.502) (width 0.254) (layer F.Cu) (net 1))
 (segment (start 144.526 79.629) (end 144.454 79.701) (width 0.254) (layer F.Cu) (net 2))
 (segment (start 144.454 79.701) (end 144.526 79.629) (width 0.254) (layer F.Cu) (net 2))
 (via (at 144.454 79.701) (size 0.6858) (drill 0.3302) (layers F.Cu B.Cu) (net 2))
 (segment (start 144.454 79.701) (end 146.431 81.678) (width 0.254) (layer B.Cu) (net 2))
 (segment (start 146.431 81.678) (end 146.431 108.839) (width 0.254) (layer B.Cu) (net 2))
 (segment (start 146.431 108.839) (end 145.161 110.109) (width 0.254) (layer B.Cu) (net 2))
 (segment (start 142.621 79.701) (end 144.454 79.701) (width 0.254) (layer F.Cu) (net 2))
 (segment (start 142.621 110.109) (end 142.621 108.839) (width 0.254) (layer B.Cu) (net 30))
 (segment (start 147.78 81.201) (end 155.321 81.201) (width 0.254) (layer F.Cu) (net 30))
 (segment (start 145.669 83.312) (end 147.78 81.201) (width 0.254) (layer F.Cu) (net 30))
 (via (at 145.669 83.312) (size 0.6858) (drill 0.3302) (layers F.Cu B.Cu) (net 30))
 (segment (start 145.669 105.791) (end 145.669 84.4804) (width 0.254) (layer B.Cu) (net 30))
 (segment (start 145.669 84.4804) (end 145.669 83.312) (width 0.254) (layer B.Cu) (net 30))
 (segment (start 142.621 108.839) (end 145.669 105.791) (width 0.254) (layer B.Cu) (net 30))
 (segment (start 149.559 104.648) (end 153.336 104.648) (width 0.254) (layer F.Cu) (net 38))
 (segment (start 149.559 104.648) (end 149.559 104.093) (width 0.254) (layer F.Cu) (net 38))
 (segment (start 149.559 104.093) (end 148.905 103.439) (width 0.254) (layer F.Cu) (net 38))
 (segment (start 148.905 103.439) (end 148.905 102.446) (width 0.254) (layer F.Cu) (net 38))
 (segment (start 155.321 78.201) (end 151.034 78.201) (width 0.254) (layer F.Cu) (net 32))
 (segment (start 151.034 78.201) (end 148.717 80.518) (width 0.254) (layer F.Cu) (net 32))
 (segment (start 148.717 80.518) (end 147.193 80.518) (width 0.254) (layer F.Cu) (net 32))
 (segment (start 147.193 80.518) (end 144.526 83.185) (width 0.254) (layer F.Cu) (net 32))
 (segment (start 143.256 107.745) (end 144.956 107.745) (width 0.254) (layer F.Cu) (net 32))
 (segment (start 154.813 108.03) (end 156.036 106.807) (width 0.254) (layer F.Cu) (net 32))
 (segment (start 154.813 108.077) (end 154.813 108.03) (width 0.254) (layer F.Cu) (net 32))
 (segment (start 154.686 108.204) (end 154.813 108.077) (width 0.254) (layer F.Cu) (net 32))
 (via (at 154.686 108.204) (size 0.6858) (drill 0.3302) (layers F.Cu B.Cu) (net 32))
 (segment (start 154.178 107.696) (end 154.686 108.204) (width 0.254) (layer B.Cu) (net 32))
 (segment (start 149.987 107.696) (end 154.178 107.696) (width 0.254) (layer B.Cu) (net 32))
 (segment (start 148.844 108.839) (end 149.987 107.696) (width 0.254) (layer B.Cu) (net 32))
 (via (at 148.844 108.839) (size 0.6858) (drill 0.3302) (layers F.Cu B.Cu) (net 32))
 (segment (start 148.844 108.712) (end 148.844 108.839) (width 0.254) (layer F.Cu) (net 32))
 (segment (start 148.59 108.458) (end 148.844 108.712) (width 0.254) (layer F.Cu) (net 32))
 (segment (start 145.669 108.458) (end 148.59 108.458) (width 0.254) (layer F.Cu) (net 32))
 (segment (start 144.956 107.745) (end 145.669 108.458) (width 0.254) (layer F.Cu) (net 32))
 (segment (start 141.019 107.745) (end 143.256 107.745) (width 0.254) (layer F.Cu) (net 32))
 (segment (start 140.97 107.696) (end 141.019 107.745) (width 0.254) (layer F.Cu) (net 32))
 (via (at 140.97 107.696) (size 0.6858) (drill 0.3302) (layers F.Cu B.Cu) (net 32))
 (segment (start 140.97 98.806) (end 140.97 107.696) (width 0.254) (layer B.Cu) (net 32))
 (segment (start 144.526 95.25) (end 140.97 98.806) (width 0.254) (layer B.Cu) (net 32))
 (via (at 144.526 95.25) (size 0.6858) (drill 0.3302) (layers F.Cu B.Cu) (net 32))
 (segment (start 144.653 95.25) (end 144.526 95.25) (width 0.254) (layer F.Cu) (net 32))
 (segment (start 144.526 95.377) (end 144.653 95.25) (width 0.254) (layer F.Cu) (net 32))
 (segment (start 144.526 83.185) (end 144.526 95.377) (width 0.254) (layer F.Cu) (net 32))
 (segment (start 155.321 82.701) (end 153.9 82.701) (width 0.254) (layer F.Cu) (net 29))
 (segment (start 157.48 100.965) (end 156.036 102.409) (width 0.254) (layer F.Cu) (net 29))
 (via (at 157.48 100.965) (size 0.6858) (drill 0.3302) (layers F.Cu B.Cu) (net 29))
 (segment (start 157.48 98.044) (end 157.48 100.965) (width 0.254) (layer B.Cu) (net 29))
 (segment (start 156.972 97.536) (end 157.48 98.044) (width 0.254) (layer B.Cu) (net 29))
 (segment (start 155.575 97.536) (end 156.972 97.536) (width 0.254) (layer B.Cu) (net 29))
 (segment (start 153.035 94.996) (end 155.575 97.536) (width 0.254) (layer B.Cu) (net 29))
 (via (at 153.035 94.996) (size 0.6858) (drill 0.3302) (layers F.Cu B.Cu) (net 29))
 (segment (start 152.908 94.869) (end 153.035 94.996) (width 0.254) (layer F.Cu) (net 29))
 (segment (start 152.908 83.693) (end 152.908 94.869) (width 0.254) (layer F.Cu) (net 29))
 (segment (start 153.9 82.701) (end 152.908 83.693) (width 0.254) (layer F.Cu) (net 29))
 (segment (start 156.036 102.409) (end 156.036 102.489) (width 0.254) (layer F.Cu) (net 29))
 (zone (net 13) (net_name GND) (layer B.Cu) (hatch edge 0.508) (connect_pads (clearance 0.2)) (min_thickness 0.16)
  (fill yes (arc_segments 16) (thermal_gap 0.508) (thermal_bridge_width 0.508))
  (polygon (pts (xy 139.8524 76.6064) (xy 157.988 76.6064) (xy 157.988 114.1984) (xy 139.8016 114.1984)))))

